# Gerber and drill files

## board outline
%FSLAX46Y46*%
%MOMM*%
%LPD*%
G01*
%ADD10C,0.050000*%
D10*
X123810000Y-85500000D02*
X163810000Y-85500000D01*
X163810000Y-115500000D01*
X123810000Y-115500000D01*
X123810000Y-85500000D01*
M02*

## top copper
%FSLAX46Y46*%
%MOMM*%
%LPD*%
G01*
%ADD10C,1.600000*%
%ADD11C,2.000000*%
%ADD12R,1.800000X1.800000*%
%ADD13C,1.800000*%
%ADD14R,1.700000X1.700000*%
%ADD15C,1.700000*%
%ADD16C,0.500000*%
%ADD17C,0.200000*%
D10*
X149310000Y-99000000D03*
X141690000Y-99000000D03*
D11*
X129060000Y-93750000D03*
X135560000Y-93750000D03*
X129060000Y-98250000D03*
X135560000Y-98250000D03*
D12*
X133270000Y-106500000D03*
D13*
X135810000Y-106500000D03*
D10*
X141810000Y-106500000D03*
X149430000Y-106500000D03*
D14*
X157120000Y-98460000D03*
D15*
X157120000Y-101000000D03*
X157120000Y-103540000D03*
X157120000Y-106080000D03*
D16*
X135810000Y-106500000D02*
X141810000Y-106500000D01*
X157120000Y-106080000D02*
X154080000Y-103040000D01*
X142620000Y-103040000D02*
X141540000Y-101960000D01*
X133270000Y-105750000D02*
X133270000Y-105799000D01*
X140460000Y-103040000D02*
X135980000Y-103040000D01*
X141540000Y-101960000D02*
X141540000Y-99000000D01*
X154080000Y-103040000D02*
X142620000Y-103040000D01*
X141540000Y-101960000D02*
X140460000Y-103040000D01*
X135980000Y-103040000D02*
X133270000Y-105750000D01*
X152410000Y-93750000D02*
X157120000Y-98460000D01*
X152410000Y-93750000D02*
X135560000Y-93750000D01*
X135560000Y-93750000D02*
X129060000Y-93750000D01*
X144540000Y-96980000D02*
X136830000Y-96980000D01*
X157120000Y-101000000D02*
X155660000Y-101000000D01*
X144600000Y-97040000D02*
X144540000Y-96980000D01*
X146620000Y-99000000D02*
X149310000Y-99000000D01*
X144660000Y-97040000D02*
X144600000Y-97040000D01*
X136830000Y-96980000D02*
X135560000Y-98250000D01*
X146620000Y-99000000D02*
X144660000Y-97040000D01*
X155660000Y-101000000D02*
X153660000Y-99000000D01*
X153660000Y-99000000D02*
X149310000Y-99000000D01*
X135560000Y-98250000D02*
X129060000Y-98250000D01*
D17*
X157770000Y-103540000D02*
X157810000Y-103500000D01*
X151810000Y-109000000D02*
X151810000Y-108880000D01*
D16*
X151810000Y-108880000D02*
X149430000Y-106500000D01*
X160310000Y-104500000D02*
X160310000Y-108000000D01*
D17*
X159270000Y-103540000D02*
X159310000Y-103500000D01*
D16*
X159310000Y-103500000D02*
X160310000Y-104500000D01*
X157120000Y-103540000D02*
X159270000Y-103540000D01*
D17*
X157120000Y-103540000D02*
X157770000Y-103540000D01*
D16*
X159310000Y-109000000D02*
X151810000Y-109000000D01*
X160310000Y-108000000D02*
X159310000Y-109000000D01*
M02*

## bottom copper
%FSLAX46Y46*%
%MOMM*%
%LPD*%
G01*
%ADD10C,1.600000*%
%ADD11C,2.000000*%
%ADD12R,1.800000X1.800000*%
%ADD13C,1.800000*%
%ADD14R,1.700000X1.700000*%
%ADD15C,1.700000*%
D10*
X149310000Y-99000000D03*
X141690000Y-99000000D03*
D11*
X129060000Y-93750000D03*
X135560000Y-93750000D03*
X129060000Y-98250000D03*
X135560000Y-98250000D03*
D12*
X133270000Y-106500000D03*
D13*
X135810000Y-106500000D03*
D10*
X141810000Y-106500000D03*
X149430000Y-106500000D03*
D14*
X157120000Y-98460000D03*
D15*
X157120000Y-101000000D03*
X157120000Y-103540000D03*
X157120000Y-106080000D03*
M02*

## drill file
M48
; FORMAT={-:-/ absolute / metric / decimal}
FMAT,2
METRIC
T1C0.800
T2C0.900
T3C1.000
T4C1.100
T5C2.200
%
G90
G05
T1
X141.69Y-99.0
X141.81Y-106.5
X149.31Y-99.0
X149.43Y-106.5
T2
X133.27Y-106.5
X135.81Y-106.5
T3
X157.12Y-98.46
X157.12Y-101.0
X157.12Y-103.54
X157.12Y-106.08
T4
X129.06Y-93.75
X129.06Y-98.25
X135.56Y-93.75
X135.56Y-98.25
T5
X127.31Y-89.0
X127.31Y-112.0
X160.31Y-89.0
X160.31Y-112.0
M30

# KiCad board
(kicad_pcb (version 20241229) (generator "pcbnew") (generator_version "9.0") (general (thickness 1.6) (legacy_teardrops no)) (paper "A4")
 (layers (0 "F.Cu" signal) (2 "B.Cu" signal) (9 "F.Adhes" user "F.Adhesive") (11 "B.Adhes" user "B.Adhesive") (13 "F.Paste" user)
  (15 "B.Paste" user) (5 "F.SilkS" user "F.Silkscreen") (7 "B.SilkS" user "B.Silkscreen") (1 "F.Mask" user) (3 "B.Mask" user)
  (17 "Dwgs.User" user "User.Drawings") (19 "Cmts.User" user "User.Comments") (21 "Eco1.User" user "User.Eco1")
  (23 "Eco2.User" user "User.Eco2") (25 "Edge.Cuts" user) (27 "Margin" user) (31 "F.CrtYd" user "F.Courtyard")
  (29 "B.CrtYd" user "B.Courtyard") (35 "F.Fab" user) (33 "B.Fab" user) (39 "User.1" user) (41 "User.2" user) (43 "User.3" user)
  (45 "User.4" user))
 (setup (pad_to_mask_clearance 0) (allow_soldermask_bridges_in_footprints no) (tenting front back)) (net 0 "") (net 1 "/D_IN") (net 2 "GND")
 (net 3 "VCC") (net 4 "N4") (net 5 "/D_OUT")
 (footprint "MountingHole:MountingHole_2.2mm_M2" (layer "F.Cu") (at 127.31 89)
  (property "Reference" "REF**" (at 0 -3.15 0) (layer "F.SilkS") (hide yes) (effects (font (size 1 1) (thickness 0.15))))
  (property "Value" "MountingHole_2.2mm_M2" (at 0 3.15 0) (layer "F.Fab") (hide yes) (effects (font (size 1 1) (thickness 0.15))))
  (pad "" np_thru_hole circle (at 0 0) (size 2.2 2.2) (drill 2.2) (layers "*.Cu" "*.Mask")))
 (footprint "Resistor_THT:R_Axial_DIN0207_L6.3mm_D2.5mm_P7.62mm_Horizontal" (layer "F.Cu") (at 149.31 99 180)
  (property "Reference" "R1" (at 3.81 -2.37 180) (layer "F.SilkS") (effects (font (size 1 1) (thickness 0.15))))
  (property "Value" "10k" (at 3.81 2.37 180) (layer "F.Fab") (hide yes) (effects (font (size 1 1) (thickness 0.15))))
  (pad "1" thru_hole circle (at 0 0 180) (size 1.6 1.6) (drill 0.8) (layers "*.Cu" "*.Mask") (remove_unused_layers no) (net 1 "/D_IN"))
  (pad "2" thru_hole circle (at 7.62 0 180) (size 1.6 1.6) (drill 0.8) (layers "*.Cu" "*.Mask") (remove_unused_layers no) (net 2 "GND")))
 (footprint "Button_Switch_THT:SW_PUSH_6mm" (layer "F.Cu") (at 129.06 93.75)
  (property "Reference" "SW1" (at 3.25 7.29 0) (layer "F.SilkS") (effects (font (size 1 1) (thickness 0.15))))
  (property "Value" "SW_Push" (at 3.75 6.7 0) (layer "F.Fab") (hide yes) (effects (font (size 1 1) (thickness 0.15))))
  (pad "1" thru_hole circle (at 0 0 90) (size 2 2) (drill 1.1) (layers "*.Cu" "*.Mask") (remove_unused_layers no) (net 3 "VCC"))
  (pad "1" thru_hole circle (at 6.5 0 90) (size 2 2) (drill 1.1) (layers "*.Cu" "*.Mask") (remove_unused_layers no) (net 3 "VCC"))
  (pad "2" thru_hole circle (at 0 4.5 90) (size 2 2) (drill 1.1) (layers "*.Cu" "*.Mask") (remove_unused_layers no) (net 1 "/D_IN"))
  (pad "2" thru_hole circle (at 6.5 4.5 90) (size 2 2) (drill 1.1) (layers "*.Cu" "*.Mask") (remove_unused_layers no) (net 1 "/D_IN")))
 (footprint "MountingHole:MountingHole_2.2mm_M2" (layer "F.Cu") (at 127.31 112)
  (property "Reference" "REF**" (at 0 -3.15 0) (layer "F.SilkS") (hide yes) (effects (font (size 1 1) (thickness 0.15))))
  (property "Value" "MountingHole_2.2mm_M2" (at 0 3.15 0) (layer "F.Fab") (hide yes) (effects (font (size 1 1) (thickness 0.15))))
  (pad "" np_thru_hole circle (at 0 0) (size 2.2 2.2) (drill 2.2) (layers "*.Cu" "*.Mask")))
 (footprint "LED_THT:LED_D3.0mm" (layer "F.Cu") (at 133.27 106.5)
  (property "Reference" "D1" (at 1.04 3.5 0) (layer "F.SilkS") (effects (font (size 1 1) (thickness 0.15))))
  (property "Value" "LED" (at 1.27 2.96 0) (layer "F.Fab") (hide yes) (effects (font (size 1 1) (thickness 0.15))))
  (pad "1" thru_hole rect (at 0 0) (size 1.8 1.8) (drill 0.9) (layers "*.Cu" "*.Mask") (remove_unused_layers no) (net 2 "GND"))
  (pad "2" thru_hole circle (at 2.54 0) (size 1.8 1.8) (drill 0.9) (layers "*.Cu" "*.Mask") (remove_unused_layers no) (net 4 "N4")))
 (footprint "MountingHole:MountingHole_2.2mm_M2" (layer "F.Cu") (at 160.31 89)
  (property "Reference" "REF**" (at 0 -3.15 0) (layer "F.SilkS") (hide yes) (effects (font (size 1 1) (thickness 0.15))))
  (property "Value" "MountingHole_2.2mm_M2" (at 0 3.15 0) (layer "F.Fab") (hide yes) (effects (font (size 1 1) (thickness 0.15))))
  (pad "" np_thru_hole circle (at 0 0) (size 2.2 2.2) (drill 2.2) (layers "*.Cu" "*.Mask")))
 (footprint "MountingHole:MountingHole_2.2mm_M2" (layer "F.Cu") (at 160.31 112)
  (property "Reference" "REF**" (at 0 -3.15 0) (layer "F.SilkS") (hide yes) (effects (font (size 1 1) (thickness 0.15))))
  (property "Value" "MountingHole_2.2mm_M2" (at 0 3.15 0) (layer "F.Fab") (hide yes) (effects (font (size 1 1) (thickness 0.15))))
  (pad "" np_thru_hole circle (at 0 0) (size 2.2 2.2) (drill 2.2) (layers "*.Cu" "*.Mask")))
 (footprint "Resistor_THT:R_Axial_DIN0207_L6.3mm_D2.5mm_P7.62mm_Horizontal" (layer "F.Cu") (at 141.81 106.5)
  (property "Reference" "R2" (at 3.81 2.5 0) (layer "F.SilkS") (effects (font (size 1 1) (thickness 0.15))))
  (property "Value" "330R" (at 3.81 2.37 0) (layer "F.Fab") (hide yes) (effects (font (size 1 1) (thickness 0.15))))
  (pad "1" thru_hole circle (at 0 0) (size 1.6 1.6) (drill 0.8) (layers "*.Cu" "*.Mask") (remove_unused_layers no) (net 4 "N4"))
  (pad "2" thru_hole circle (at 7.62 0) (size 1.6 1.6) (drill 0.8) (layers "*.Cu" "*.Mask") (remove_unused_layers no) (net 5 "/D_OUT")))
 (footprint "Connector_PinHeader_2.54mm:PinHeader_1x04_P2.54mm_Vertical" (layer "F.Cu") (at 157.12 98.46)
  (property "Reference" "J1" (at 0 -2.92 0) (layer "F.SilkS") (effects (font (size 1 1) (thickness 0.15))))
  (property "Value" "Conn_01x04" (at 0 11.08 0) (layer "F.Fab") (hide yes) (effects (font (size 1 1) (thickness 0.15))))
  (pad "1" thru_hole rect (at 0 0) (size 1.7 1.7) (drill 1) (layers "*.Cu" "*.Mask") (remove_unused_layers no) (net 3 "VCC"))
  (pad "2" thru_hole circle (at 0 2.54) (size 1.7 1.7) (drill 1) (layers "*.Cu" "*.Mask") (remove_unused_layers no) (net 1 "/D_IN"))
  (pad "3" thru_hole circle (at 0 5.08) (size 1.7 1.7) (drill 1) (layers "*.Cu" "*.Mask") (remove_unused_layers no) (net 5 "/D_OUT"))
  (pad "4" thru_hole circle (at 0 7.62) (size 1.7 1.7) (drill 1) (layers "*.Cu" "*.Mask") (remove_unused_layers no) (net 2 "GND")))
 (gr_rect (start 123.81 85.5) (end 163.81 115.5) (stroke (width 0.05) (type solid)) (fill no) (layer "Edge.Cuts"))
 (segment (start 135.81 106.5) (end 141.81 106.5) (width 0.5) (layer "F.Cu") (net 4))
 (segment (start 157.12 106.08) (end 154.08 103.04) (width 0.5) (layer "F.Cu") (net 2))
 (segment (start 142.62 103.04) (end 141.54 101.96) (width 0.5) (layer "F.Cu") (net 2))
 (segment (start 133.27 105.75) (end 133.27 105.799) (width 0.5) (layer "F.Cu") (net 2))
 (segment (start 140.46 103.04) (end 135.98 103.04) (width 0.5) (layer "F.Cu") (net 2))
 (segment (start 141.54 101.96) (end 141.54 99) (width 0.5) (layer "F.Cu") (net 2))
 (segment (start 154.08 103.04) (end 142.62 103.04) (width 0.5) (layer "F.Cu") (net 2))
 (segment (start 141.54 101.96) (end 140.46 103.04) (width 0.5) (layer "F.Cu") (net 2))
 (segment (start 135.98 103.04) (end 133.27 105.75) (width 0.5) (layer "F.Cu") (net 2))
 (segment (start 152.41 93.75) (end 157.12 98.46) (width 0.5) (layer "F.Cu") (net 3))
 (segment (start 152.41 93.75) (end 135.56 93.75) (width 0.5) (layer "F.Cu") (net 3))
 (segment (start 135.56 93.75) (end 129.06 93.75) (width 0.5) (layer "F.Cu") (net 3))
 (segment (start 144.54 96.98) (end 136.83 96.98) (width 0.5) (layer "F.Cu") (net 1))
 (segment (start 157.12 101) (end 155.66 101) (width 0.5) (layer "F.Cu") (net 1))
 (segment (start 144.6 97.04) (end 144.54 96.98) (width 0.5) (layer "F.Cu") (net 1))
 (segment (start 146.62 99) (end 149.31 99) (width 0.5) (layer "F.Cu") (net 1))
 (segment (start 144.66 97.04) (end 144.6 97.04) (width 0.5) (layer "F.Cu") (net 1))
 (segment (start 136.83 96.98) (end 135.56 98.25) (width 0.5) (layer "F.Cu") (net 1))
 (segment (start 146.62 99) (end 144.66 97.04) (width 0.5) (layer "F.Cu") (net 1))
 (segment (start 155.66 101) (end 153.66 99) (width 0.5) (layer "F.Cu") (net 1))
 (segment (start 153.66 99) (end 149.31 99) (width 0.5) (layer "F.Cu") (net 1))
 (segment (start 135.56 98.25) (end 129.06 98.25) (width 0.5) (layer "F.Cu") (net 1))
 (segment (start 157.77 103.54) (end 157.81 103.5) (width 0.2) (layer "F.Cu") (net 5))
 (segment (start 151.81 109) (end 151.81 108.88) (width 0.2) (layer "F.Cu") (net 5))
 (segment (start 151.81 108.88) (end 149.43 106.5) (width 0.5) (layer "F.Cu") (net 5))
 (segment (start 160.31 104.5) (end 160.31 108) (width 0.5) (layer "F.Cu") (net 5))
 (segment (start 159.27 103.54) (end 159.31 103.5) (width 0.2) (layer "F.Cu") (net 5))
 (segment (start 159.31 103.5) (end 160.31 104.5) (width 0.5) (layer "F.Cu") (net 5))
 (segment (start 157.12 103.54) (end 159.27 103.54) (width 0.5) (layer "F.Cu") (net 5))
 (segment (start 157.12 103.54) (end 157.77 103.54) (width 0.2) (layer "F.Cu") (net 5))
 (segment (start 159.31 109) (end 151.81 109) (width 0.5) (layer "F.Cu") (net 5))
 (segment (start 160.31 108) (end 159.31 109) (width 0.5) (layer "F.Cu") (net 5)))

